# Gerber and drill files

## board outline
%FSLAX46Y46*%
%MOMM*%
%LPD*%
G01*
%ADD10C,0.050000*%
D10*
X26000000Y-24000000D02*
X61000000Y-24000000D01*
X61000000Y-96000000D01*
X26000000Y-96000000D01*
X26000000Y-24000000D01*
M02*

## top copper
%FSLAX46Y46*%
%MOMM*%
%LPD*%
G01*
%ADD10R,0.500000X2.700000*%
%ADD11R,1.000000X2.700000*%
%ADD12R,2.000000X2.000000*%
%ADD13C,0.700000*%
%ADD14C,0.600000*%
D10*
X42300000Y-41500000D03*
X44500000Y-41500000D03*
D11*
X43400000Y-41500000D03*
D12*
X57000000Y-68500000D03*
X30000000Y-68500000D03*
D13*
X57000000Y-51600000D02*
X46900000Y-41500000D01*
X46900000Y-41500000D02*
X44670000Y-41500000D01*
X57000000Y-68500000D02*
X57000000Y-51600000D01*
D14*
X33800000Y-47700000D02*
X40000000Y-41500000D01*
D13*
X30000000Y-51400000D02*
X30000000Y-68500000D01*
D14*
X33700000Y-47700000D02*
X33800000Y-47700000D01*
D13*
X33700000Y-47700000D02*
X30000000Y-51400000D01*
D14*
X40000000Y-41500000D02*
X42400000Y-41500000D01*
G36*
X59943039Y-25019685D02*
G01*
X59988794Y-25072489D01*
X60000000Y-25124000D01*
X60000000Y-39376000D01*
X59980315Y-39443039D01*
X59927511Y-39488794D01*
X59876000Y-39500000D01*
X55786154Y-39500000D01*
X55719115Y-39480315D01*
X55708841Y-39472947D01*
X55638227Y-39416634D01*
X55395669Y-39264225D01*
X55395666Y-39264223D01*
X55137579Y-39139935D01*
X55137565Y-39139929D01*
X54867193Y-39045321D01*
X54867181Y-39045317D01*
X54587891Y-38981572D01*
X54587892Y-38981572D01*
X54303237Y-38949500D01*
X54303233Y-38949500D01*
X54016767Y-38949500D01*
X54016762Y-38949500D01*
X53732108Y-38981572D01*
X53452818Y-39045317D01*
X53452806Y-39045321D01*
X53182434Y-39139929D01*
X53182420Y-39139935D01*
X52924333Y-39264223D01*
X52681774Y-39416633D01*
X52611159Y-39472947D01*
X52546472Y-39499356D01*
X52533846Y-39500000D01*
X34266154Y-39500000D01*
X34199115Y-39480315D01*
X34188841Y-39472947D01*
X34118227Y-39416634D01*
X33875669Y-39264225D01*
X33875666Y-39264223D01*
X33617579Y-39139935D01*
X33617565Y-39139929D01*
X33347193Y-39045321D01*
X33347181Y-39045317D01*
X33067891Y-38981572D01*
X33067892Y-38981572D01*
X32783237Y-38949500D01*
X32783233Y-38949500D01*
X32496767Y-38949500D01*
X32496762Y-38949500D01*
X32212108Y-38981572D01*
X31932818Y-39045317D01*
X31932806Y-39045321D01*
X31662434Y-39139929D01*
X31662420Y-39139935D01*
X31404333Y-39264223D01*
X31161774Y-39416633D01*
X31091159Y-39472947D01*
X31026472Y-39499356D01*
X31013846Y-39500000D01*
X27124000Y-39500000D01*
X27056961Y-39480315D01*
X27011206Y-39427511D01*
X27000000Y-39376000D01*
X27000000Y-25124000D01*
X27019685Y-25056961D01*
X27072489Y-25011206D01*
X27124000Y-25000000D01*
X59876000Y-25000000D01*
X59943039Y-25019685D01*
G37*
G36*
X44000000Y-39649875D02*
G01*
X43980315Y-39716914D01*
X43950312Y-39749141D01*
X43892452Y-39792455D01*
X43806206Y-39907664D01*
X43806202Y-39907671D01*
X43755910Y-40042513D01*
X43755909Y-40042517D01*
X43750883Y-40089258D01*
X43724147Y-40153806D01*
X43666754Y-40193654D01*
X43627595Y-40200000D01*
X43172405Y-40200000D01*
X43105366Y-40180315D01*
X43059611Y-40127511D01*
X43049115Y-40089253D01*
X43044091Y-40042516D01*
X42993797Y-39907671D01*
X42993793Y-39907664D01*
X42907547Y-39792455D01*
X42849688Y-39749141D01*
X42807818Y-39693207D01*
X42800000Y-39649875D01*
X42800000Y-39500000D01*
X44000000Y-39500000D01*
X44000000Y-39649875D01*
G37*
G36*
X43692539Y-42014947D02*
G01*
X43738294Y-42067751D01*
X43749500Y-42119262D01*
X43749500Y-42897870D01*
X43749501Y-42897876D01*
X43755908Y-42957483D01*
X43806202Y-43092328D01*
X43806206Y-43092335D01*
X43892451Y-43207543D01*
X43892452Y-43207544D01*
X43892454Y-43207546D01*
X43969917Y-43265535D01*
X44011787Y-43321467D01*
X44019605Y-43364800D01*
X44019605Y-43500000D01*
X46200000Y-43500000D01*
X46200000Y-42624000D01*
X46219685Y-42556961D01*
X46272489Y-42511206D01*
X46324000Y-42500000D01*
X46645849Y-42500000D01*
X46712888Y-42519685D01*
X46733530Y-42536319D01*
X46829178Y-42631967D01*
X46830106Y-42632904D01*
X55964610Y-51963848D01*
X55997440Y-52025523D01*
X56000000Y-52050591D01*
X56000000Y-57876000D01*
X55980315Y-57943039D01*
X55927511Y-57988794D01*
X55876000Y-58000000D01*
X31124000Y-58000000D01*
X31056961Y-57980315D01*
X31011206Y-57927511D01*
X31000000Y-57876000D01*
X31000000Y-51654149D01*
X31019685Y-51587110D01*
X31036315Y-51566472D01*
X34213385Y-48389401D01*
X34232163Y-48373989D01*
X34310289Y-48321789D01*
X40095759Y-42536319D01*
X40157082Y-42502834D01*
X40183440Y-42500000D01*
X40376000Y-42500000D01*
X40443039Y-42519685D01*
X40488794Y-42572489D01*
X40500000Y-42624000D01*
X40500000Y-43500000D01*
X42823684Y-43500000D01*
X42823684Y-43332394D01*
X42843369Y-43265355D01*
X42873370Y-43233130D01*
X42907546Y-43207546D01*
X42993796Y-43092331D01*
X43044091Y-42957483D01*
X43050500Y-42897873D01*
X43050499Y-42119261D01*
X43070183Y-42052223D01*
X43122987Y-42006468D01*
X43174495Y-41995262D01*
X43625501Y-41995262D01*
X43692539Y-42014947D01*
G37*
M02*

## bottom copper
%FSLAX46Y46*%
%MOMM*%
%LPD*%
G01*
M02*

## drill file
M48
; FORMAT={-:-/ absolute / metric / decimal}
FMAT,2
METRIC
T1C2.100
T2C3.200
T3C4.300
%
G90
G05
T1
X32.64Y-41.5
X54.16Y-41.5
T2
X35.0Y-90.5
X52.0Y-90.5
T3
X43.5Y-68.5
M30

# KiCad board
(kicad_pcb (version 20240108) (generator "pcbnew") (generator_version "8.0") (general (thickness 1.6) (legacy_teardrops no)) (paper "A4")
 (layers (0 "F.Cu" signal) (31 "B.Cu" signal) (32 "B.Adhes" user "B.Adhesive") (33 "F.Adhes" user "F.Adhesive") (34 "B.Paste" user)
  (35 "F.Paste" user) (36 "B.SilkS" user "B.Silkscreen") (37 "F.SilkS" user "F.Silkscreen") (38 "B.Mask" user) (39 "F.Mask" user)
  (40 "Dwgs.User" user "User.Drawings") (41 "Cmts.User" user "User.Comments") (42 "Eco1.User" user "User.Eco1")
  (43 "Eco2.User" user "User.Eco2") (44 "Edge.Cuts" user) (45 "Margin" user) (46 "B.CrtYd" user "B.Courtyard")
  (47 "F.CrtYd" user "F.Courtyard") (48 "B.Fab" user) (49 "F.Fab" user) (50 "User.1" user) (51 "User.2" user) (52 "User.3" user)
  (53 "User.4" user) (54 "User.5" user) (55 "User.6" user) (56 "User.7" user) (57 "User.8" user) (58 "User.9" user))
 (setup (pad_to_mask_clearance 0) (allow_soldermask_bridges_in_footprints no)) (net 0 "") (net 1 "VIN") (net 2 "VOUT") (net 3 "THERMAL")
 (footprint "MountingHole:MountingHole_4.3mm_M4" (layer "F.Cu") (at 43.5 68.5)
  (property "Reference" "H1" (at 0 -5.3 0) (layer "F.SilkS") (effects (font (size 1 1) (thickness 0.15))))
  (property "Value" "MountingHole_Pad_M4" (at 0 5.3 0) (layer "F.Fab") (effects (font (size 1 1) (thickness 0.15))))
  (pad "" np_thru_hole circle (at 0 0) (size 4.3 4.3) (drill 4.3) (layers "*.Cu" "*.Mask")))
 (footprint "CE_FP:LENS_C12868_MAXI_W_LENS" (layer "F.Cu") (at 43.4 41.5)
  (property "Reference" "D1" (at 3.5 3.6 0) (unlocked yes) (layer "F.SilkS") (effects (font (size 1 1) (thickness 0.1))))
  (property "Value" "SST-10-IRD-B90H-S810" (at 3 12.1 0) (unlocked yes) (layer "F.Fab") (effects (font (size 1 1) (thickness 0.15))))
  (pad "" np_thru_hole circle (at -10.76 0) (size 2.1 2.1) (drill 2.1) (layers "F&B.Cu" "*.Mask") (clearance 1.5))
  (pad "" np_thru_hole circle (at 10.76 0) (size 2.1 2.1) (drill 2.1) (layers "F&B.Cu" "*.Mask") (clearance 1.5))
  (pad "A" smd rect (at -1.1 0 180) (size 0.5 2.7) (layers "F.Cu" "F.Paste" "F.Mask") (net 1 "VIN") (solder_mask_margin 0.102))
  (pad "C" smd rect (at 1.1 0 180) (size 0.5 2.7) (layers "F.Cu" "F.Paste" "F.Mask") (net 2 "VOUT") (solder_mask_margin 0.102))
  (pad "S" smd rect (at 0 0 180) (size 1 2.7) (layers "F.Cu" "F.Mask") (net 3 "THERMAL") (solder_mask_margin 0.102)))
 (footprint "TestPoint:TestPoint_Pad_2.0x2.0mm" (layer "F.Cu") (at 57 68.5)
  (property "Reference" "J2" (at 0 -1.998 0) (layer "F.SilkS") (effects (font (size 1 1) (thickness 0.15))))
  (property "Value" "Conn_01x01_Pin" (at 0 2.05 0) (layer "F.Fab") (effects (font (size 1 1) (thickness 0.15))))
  (pad "1" smd rect (at 0 0) (size 2 2) (layers "F.Cu" "F.Mask") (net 2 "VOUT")))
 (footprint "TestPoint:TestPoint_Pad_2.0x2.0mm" (layer "F.Cu") (at 30 68.5)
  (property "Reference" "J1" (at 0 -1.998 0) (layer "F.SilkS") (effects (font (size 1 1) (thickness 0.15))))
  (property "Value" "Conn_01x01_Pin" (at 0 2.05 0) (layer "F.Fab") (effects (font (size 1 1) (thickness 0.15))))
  (pad "1" smd rect (at 0 0) (size 2 2) (layers "F.Cu" "F.Mask") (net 1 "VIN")))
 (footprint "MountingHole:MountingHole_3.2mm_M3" (layer "F.Cu") (at 35 90.5)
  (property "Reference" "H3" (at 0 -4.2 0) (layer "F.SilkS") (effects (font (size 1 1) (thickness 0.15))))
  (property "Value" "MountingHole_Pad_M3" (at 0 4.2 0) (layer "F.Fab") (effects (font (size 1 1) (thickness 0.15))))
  (pad "" np_thru_hole circle (at 0 0) (size 3.2 3.2) (drill 3.2) (layers "*.Cu" "*.Mask")))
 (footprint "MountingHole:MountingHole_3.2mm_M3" (layer "F.Cu") (at 52 90.5)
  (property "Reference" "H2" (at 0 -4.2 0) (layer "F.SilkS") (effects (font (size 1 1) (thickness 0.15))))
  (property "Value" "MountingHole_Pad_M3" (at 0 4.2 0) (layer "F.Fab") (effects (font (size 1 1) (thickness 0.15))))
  (pad "" np_thru_hole circle (at 0 0) (size 3.2 3.2) (drill 3.2) (layers "*.Cu" "*.Mask")))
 (gr_rect (start 26 24) (end 61 96) (stroke (width 0.05) (type default)) (fill none) (layer "Edge.Cuts"))
 (segment (start 57 51.6) (end 46.9 41.5) (width 0.7) (layer "F.Cu") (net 2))
 (segment (start 46.9 41.5) (end 44.67 41.5) (width 0.7) (layer "F.Cu") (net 2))
 (segment (start 57 68.5) (end 57 51.6) (width 0.7) (layer "F.Cu") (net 2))
 (segment (start 33.8 47.7) (end 40 41.5) (width 0.6) (layer "F.Cu") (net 1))
 (segment (start 30 51.4) (end 30 68.5) (width 0.7) (layer "F.Cu") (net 1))
 (segment (start 33.7 47.7) (end 33.8 47.7) (width 0.6) (layer "F.Cu") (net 1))
 (segment (start 33.7 47.7) (end 30 51.4) (width 0.7) (layer "F.Cu") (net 1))
 (segment (start 40 41.5) (end 42.4 41.5) (width 0.6) (layer "F.Cu") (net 1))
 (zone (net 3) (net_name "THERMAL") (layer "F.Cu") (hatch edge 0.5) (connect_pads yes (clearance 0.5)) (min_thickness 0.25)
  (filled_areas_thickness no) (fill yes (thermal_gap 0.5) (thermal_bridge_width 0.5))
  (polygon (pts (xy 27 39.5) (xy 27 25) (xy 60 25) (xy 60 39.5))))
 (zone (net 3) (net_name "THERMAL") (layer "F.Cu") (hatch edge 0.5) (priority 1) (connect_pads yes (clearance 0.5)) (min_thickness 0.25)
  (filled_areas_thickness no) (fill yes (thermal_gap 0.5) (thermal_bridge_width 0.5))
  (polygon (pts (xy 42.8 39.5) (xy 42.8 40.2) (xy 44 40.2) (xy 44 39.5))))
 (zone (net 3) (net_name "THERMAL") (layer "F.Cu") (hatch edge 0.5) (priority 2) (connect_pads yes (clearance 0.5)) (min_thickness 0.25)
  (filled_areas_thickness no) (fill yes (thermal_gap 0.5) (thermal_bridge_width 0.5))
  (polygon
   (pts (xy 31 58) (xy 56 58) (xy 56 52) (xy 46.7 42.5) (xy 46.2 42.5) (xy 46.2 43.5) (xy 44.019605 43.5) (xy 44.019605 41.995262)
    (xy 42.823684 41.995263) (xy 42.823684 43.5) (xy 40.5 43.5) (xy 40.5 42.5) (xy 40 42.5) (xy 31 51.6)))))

